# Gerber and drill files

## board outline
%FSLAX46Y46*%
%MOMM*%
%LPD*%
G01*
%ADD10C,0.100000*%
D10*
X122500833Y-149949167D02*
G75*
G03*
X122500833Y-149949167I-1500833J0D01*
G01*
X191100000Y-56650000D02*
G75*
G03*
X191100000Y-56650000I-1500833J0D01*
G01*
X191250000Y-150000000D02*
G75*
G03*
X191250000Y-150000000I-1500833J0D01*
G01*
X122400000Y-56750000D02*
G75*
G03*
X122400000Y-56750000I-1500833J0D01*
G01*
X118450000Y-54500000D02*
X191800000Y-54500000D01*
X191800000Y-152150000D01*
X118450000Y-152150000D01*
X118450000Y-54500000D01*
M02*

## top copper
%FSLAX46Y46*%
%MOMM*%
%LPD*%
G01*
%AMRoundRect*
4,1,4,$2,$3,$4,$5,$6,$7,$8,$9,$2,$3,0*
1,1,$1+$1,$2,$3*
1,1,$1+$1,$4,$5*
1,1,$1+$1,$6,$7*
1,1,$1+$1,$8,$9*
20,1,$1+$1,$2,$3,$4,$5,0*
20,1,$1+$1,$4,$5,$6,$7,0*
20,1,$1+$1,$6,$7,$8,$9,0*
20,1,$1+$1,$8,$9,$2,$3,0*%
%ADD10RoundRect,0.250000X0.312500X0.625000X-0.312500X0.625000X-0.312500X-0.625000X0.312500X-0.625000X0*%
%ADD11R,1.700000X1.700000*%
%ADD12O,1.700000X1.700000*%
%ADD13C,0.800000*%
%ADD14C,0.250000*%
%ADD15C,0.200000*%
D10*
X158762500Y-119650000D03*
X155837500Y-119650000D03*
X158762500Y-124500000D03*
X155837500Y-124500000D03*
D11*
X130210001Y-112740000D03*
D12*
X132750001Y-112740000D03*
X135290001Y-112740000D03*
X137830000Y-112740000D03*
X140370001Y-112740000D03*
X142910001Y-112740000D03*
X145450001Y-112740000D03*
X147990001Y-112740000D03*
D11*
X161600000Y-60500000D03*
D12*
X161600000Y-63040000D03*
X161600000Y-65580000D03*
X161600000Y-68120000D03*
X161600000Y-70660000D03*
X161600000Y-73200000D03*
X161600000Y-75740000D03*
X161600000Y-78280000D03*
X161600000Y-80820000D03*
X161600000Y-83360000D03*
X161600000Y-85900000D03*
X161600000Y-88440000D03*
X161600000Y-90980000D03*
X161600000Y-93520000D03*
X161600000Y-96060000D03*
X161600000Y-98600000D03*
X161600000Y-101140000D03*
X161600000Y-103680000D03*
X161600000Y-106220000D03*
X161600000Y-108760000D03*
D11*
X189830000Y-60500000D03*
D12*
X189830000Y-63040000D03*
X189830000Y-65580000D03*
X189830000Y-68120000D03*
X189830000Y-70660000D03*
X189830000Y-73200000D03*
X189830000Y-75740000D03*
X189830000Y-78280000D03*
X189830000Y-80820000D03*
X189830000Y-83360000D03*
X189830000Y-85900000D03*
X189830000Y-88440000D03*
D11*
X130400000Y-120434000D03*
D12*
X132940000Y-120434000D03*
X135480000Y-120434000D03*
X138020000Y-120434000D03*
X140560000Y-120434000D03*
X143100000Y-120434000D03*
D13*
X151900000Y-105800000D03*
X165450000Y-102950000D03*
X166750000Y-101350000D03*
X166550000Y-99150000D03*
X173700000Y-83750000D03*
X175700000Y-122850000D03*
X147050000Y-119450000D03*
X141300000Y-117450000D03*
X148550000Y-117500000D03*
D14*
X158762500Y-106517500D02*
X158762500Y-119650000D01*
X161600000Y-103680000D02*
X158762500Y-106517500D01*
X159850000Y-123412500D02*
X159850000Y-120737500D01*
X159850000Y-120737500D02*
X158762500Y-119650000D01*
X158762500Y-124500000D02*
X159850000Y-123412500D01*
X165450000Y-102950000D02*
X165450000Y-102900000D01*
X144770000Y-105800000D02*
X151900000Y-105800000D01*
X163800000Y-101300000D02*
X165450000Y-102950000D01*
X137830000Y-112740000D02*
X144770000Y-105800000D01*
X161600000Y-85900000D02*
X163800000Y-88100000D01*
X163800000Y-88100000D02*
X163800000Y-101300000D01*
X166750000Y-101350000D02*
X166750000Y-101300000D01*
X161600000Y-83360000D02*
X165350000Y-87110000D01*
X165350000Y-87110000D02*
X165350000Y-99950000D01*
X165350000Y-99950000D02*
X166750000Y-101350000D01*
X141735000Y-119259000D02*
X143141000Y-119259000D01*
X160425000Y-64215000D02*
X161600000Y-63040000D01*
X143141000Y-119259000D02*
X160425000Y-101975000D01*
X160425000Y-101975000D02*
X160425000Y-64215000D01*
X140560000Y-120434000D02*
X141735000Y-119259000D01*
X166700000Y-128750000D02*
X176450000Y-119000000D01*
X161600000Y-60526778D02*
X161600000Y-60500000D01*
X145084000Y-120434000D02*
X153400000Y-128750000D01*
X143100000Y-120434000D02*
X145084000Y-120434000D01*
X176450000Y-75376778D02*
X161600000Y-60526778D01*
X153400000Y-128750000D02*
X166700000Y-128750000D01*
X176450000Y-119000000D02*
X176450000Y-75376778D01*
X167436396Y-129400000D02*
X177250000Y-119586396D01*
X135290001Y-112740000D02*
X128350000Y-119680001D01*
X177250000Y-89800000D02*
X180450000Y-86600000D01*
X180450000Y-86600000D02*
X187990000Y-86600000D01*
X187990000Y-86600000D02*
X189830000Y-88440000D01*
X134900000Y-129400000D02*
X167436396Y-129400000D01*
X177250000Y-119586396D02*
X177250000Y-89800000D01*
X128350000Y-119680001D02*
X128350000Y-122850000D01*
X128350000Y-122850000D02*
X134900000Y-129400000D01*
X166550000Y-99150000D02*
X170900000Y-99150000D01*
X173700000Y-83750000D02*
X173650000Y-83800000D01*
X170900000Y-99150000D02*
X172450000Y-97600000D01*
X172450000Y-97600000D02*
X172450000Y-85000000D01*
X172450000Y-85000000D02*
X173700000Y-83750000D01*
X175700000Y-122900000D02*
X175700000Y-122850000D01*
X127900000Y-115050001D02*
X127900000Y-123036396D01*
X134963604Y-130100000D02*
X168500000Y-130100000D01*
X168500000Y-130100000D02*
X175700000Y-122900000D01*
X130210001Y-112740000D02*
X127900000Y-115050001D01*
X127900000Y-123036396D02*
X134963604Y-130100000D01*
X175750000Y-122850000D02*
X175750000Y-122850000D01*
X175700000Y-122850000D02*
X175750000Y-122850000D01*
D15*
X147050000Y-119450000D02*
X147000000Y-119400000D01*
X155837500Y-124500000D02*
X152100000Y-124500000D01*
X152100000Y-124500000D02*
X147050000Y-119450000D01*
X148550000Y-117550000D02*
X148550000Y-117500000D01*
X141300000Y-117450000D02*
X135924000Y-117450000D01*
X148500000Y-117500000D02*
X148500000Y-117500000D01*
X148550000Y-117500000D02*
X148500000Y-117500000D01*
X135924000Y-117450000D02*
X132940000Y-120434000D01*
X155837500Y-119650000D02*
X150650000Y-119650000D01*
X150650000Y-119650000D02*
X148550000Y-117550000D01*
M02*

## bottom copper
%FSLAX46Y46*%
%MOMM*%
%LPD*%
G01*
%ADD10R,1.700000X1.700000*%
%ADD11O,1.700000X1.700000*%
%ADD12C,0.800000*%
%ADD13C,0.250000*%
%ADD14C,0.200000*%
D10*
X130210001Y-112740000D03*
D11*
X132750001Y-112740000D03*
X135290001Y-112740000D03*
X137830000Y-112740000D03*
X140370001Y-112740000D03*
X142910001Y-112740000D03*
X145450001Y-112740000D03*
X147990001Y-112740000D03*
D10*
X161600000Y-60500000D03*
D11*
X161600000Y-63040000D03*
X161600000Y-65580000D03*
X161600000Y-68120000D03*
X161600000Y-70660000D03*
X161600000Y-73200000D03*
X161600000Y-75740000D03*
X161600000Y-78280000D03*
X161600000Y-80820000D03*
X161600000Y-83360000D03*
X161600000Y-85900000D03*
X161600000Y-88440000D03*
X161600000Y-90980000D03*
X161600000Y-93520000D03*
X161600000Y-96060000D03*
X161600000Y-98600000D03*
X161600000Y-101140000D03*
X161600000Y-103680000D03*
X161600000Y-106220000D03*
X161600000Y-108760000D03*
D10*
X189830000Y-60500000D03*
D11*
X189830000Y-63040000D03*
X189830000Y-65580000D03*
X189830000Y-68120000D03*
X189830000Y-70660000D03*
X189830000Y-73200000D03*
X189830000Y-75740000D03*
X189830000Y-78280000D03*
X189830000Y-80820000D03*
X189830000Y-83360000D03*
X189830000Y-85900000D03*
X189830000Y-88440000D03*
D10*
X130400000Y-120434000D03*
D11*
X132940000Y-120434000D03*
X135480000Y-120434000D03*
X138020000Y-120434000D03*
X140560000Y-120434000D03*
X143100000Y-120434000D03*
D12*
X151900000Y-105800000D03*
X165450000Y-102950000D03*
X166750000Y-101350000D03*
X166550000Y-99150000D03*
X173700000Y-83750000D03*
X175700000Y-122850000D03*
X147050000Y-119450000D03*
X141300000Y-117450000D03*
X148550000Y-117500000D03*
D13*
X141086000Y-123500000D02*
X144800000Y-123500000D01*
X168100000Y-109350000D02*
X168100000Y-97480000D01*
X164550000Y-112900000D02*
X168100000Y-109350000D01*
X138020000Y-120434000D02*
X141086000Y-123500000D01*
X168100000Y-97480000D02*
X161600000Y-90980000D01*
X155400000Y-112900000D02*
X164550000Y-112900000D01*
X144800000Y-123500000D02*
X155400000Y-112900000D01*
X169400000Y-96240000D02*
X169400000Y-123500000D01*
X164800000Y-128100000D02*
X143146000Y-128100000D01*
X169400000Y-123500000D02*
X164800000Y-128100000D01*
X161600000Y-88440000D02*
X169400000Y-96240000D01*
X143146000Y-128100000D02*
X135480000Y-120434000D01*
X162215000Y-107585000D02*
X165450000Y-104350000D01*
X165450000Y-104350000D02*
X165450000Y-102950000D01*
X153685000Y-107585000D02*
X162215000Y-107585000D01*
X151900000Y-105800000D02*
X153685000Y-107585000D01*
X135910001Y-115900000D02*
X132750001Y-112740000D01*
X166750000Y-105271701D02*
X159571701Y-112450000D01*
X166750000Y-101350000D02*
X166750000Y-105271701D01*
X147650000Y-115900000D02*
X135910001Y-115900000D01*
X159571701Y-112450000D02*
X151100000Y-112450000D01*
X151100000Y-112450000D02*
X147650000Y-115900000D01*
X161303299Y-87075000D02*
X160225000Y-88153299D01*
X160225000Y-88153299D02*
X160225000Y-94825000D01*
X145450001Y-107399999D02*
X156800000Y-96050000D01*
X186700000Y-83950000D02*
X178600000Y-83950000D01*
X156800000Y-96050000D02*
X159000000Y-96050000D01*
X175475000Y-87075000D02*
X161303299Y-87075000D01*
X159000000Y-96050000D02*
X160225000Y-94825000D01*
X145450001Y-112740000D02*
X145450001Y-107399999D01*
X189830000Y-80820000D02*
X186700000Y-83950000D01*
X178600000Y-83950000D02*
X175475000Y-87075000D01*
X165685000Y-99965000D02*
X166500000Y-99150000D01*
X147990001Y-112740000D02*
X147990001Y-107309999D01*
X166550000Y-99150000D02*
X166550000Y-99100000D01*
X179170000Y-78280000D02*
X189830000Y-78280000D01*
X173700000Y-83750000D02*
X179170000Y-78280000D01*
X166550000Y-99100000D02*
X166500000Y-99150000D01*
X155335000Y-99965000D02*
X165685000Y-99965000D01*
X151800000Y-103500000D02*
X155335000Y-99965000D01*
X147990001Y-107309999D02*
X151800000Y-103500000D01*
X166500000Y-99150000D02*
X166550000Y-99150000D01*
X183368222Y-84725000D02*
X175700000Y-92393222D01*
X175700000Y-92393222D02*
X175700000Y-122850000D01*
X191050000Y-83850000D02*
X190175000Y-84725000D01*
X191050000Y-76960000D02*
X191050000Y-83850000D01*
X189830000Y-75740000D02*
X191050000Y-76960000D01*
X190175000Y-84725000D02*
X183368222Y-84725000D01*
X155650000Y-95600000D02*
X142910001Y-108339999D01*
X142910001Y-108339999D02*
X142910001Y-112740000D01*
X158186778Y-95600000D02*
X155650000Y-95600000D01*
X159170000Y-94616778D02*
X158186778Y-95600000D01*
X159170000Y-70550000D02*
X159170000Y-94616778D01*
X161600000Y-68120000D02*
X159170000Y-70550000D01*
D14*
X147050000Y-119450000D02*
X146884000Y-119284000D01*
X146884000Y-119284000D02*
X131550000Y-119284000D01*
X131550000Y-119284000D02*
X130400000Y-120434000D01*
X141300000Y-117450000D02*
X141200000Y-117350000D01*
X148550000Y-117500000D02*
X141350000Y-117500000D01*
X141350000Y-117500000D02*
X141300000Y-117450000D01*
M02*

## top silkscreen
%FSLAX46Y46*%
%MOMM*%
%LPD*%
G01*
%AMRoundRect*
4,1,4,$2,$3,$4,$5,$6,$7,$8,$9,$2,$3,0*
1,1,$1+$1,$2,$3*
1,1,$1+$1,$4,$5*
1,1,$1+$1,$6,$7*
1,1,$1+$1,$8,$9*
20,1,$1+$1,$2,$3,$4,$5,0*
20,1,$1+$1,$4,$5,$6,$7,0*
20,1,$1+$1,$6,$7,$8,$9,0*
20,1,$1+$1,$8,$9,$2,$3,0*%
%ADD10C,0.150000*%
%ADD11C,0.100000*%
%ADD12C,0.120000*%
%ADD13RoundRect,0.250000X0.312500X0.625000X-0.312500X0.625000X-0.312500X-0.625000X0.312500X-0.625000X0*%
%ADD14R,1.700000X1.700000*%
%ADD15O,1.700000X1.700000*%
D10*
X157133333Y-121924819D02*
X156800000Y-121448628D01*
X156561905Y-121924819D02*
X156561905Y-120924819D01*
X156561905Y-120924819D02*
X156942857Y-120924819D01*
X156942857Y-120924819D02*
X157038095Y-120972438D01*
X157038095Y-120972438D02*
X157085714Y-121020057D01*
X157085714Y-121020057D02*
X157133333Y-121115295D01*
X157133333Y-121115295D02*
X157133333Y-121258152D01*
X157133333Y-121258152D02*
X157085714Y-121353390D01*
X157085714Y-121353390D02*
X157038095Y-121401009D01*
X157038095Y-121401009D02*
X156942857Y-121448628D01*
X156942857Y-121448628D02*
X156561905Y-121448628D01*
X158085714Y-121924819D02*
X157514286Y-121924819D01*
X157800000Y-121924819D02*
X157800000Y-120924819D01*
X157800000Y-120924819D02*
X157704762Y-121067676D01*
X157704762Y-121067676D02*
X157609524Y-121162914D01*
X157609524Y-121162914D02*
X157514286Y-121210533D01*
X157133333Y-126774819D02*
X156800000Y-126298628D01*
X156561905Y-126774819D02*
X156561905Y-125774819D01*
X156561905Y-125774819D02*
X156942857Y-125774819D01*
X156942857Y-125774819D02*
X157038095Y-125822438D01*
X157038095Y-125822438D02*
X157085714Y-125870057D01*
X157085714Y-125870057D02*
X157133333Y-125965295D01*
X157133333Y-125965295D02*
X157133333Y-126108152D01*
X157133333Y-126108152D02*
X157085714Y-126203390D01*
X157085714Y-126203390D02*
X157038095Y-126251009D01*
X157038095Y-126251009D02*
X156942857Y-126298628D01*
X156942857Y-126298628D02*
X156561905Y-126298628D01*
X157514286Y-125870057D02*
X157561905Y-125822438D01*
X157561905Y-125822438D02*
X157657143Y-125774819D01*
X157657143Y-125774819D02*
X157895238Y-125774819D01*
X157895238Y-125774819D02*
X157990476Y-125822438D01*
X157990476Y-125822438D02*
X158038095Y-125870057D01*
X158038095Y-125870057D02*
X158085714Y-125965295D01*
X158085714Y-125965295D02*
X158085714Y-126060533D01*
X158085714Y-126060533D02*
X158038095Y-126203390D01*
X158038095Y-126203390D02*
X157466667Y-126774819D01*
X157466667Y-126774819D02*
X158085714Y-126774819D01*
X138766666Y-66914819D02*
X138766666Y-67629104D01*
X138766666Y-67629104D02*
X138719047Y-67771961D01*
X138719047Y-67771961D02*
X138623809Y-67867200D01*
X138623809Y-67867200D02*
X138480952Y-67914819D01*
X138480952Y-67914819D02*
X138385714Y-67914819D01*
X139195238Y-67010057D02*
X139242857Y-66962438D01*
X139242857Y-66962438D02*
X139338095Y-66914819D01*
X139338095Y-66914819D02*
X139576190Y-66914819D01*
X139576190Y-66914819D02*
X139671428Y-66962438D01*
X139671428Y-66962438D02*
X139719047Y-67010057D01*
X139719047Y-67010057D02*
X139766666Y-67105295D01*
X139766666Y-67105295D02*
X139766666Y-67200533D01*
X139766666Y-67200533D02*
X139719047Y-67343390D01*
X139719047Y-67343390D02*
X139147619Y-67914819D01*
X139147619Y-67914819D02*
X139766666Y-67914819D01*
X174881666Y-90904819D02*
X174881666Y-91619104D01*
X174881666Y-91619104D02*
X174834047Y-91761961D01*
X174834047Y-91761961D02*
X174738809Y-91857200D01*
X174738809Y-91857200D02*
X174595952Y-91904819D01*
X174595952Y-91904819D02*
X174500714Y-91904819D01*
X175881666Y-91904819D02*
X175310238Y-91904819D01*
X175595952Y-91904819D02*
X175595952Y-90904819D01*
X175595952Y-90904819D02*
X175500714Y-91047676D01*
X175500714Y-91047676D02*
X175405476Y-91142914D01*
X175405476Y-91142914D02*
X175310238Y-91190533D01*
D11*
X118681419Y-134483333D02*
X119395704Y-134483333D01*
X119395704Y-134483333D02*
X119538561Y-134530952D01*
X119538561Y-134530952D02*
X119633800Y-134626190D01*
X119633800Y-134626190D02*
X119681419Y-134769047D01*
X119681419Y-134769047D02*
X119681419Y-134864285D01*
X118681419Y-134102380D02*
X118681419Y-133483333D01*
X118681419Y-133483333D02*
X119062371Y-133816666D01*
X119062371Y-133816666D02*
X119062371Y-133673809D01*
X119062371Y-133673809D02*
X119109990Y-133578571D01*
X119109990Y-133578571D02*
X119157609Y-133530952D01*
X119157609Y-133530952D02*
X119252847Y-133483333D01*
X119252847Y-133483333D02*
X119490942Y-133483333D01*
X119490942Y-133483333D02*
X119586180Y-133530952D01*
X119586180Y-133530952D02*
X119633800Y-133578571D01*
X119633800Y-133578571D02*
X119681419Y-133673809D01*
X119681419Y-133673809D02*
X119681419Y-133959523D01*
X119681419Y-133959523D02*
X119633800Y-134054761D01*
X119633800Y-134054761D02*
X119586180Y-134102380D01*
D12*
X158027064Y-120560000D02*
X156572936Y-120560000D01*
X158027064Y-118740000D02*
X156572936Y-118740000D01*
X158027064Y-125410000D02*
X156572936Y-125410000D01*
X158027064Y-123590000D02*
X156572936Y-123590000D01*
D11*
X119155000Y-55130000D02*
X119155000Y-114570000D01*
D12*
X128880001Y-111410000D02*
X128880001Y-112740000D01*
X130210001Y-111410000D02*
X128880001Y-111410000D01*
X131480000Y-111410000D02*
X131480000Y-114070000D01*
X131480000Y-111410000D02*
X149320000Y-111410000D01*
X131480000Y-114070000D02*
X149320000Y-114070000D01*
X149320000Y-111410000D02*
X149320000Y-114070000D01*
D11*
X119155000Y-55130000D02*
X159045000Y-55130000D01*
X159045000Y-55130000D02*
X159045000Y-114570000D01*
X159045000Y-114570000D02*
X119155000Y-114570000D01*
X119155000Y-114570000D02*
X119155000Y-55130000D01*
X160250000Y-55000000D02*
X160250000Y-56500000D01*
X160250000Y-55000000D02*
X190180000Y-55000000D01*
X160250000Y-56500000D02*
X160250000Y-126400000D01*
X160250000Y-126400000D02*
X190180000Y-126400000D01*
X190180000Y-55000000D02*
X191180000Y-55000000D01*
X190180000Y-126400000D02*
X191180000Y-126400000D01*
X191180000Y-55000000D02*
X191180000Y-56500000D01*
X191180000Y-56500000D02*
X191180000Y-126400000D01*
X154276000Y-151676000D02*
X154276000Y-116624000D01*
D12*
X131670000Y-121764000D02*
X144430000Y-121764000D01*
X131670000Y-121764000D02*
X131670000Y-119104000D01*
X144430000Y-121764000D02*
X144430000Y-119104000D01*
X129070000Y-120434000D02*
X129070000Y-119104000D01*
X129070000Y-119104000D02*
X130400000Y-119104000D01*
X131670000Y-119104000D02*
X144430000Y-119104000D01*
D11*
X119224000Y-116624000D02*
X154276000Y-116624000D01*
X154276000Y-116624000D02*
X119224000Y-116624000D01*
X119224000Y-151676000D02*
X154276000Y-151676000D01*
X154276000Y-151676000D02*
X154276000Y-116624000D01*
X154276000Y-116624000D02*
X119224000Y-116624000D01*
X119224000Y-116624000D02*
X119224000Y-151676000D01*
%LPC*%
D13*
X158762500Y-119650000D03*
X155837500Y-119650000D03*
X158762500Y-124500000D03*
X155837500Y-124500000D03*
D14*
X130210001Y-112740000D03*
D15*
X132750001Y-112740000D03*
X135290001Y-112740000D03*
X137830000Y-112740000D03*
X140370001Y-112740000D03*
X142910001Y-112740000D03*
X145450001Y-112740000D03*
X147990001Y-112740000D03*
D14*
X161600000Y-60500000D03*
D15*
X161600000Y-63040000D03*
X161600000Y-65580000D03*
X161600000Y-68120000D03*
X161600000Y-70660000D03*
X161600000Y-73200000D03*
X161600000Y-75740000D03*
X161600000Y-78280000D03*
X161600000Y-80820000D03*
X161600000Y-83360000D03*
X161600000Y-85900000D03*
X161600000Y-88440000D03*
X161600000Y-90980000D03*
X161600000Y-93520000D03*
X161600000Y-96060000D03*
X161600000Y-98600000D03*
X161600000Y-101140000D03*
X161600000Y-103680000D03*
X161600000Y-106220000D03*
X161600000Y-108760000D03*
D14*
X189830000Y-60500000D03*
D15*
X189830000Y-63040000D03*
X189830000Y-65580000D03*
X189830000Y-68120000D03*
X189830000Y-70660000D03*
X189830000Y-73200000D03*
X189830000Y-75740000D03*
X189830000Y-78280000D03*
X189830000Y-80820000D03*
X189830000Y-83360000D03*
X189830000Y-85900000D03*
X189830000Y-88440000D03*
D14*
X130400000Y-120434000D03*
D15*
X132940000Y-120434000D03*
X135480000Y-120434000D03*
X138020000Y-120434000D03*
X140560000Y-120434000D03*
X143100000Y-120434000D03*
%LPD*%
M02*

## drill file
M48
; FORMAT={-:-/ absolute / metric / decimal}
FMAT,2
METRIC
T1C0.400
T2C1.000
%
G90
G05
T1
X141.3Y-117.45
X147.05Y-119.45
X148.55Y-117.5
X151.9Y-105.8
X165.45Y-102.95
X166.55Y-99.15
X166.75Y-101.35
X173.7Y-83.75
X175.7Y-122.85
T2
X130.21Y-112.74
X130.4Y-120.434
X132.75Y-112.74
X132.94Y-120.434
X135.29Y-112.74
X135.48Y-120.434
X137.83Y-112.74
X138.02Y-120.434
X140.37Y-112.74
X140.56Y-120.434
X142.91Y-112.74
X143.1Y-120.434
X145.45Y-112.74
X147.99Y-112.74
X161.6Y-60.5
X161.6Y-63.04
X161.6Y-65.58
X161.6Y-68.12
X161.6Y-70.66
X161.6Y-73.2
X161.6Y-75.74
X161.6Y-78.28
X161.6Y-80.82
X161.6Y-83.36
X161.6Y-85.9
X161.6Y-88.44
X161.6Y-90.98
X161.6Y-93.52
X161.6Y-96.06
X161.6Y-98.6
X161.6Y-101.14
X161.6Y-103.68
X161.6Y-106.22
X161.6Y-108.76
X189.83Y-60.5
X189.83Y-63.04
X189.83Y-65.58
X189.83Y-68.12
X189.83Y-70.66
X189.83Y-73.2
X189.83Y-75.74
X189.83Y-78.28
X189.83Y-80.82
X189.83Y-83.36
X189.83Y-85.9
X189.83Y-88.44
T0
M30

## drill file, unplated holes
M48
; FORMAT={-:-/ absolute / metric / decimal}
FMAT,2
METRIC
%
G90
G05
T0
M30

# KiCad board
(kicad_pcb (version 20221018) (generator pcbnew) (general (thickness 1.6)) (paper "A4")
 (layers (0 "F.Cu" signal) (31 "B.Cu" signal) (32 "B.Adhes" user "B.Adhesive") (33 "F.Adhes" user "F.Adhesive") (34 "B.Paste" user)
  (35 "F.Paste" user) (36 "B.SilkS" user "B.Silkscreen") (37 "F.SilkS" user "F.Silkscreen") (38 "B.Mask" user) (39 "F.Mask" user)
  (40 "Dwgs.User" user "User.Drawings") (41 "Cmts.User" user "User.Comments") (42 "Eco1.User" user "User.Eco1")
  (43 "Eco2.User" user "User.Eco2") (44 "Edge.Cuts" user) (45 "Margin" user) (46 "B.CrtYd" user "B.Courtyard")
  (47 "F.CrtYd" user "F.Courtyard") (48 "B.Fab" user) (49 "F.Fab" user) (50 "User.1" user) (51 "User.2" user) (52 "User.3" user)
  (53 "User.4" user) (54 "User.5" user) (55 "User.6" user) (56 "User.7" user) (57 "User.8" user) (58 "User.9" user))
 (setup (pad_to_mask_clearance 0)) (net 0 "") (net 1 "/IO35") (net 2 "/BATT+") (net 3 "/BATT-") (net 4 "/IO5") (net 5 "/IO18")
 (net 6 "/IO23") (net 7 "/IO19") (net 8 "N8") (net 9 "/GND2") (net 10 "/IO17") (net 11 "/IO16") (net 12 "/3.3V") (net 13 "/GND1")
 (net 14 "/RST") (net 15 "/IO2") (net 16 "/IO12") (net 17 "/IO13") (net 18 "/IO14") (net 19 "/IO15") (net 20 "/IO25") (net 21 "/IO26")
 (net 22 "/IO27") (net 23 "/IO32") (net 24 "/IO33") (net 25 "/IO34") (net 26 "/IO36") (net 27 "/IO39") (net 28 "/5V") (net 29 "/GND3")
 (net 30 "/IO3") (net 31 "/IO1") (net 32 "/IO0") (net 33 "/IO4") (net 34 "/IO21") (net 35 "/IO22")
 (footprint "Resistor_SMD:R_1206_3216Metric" (layer "F.Cu") (at 157.3 119.65 180)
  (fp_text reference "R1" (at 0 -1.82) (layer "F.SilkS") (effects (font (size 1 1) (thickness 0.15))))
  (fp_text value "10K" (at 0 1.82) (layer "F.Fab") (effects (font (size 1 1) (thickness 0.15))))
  (fp_line (start -0.727064 -0.91) (end 0.727064 -0.91) (stroke (width 0.12) (type solid)) (layer "F.SilkS"))
  (fp_line (start -0.727064 0.91) (end 0.727064 0.91) (stroke (width 0.12) (type solid)) (layer "F.SilkS"))
  (pad "1" smd roundrect (at -1.4625 0 180) (size 1.125 1.75) (layers "F.Cu" "F.Paste" "F.Mask") (roundrect_rratio 0.2222222222)
   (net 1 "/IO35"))
  (pad "2" smd roundrect (at 1.4625 0 180) (size 1.125 1.75) (layers "F.Cu" "F.Paste" "F.Mask") (roundrect_rratio 0.2222222222)
   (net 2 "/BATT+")))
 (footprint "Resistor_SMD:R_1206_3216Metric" (layer "F.Cu") (at 157.3 124.5 180)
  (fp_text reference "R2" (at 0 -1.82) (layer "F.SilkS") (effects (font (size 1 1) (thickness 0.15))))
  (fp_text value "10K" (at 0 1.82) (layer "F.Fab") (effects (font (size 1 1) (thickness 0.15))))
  (fp_line (start -0.727064 -0.91) (end 0.727064 -0.91) (stroke (width 0.12) (type solid)) (layer "F.SilkS"))
  (fp_line (start -0.727064 0.91) (end 0.727064 0.91) (stroke (width 0.12) (type solid)) (layer "F.SilkS"))
  (pad "1" smd roundrect (at -1.4625 0 180) (size 1.125 1.75) (layers "F.Cu" "F.Paste" "F.Mask") (roundrect_rratio 0.2222222222)
   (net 1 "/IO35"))
  (pad "2" smd roundrect (at 1.4625 0 180) (size 1.125 1.75) (layers "F.Cu" "F.Paste" "F.Mask") (roundrect_rratio 0.2222222222)
   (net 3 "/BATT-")))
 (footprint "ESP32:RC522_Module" (layer "F.Cu") (at 139.1 84.85)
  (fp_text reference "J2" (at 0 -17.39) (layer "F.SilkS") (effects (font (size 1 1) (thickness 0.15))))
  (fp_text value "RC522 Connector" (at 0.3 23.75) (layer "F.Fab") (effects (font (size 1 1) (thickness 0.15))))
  (fp_line (start -19.945 -29.72) (end -19.945 29.72) (stroke (width 0.1) (type default)) (layer "F.SilkS"))
  (fp_line (start -10.219999 26.56) (end -10.219999 27.89) (stroke (width 0.12) (type solid)) (layer "F.SilkS"))
  (fp_line (start -8.889999 26.56) (end -10.219999 26.56) (stroke (width 0.12) (type solid)) (layer "F.SilkS"))
  (fp_line (start -7.62 26.56) (end -7.62 29.22) (stroke (width 0.12) (type solid)) (layer "F.SilkS"))
  (fp_line (start -7.62 26.56) (end 10.22 26.56) (stroke (width 0.12) (type solid)) (layer "F.SilkS"))
  (fp_line (start -7.62 29.22) (end 10.22 29.22) (stroke (width 0.12) (type solid)) (layer "F.SilkS"))
  (fp_line (start 10.22 26.56) (end 10.22 29.22) (stroke (width 0.12) (type solid)) (layer "F.SilkS"))
  (fp_rect (start -19.945 -29.72) (end 19.945 29.72) (stroke (width 0.1) (type default)) (fill none) (layer "F.SilkS"))
  (pad "1" thru_hole rect (at -8.889999 27.89 90) (size 1.7 1.7) (drill 1) (layers "*.Cu" "*.Mask") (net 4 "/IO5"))
  (pad "2" thru_hole oval (at -6.349999 27.89 90) (size 1.7 1.7) (drill 1) (layers "*.Cu" "*.Mask") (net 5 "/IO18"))
  (pad "3" thru_hole oval (at -3.809999 27.89 90) (size 1.7 1.7) (drill 1) (layers "*.Cu" "*.Mask") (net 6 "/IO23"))
  (pad "4" thru_hole oval (at -1.27 27.89 90) (size 1.7 1.7) (drill 1) (layers "*.Cu" "*.Mask") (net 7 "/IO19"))
  (pad "5" thru_hole oval (at 1.270001 27.89 90) (size 1.7 1.7) (drill 1) (layers "*.Cu" "*.Mask") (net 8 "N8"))
  (pad "6" thru_hole oval (at 3.810001 27.89 90) (size 1.7 1.7) (drill 1) (layers "*.Cu" "*.Mask") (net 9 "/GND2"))
  (pad "7" thru_hole oval (at 6.350001 27.89 90) (size 1.7 1.7) (drill 1) (layers "*.Cu" "*.Mask") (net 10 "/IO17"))
  (pad "8" thru_hole oval (at 8.890001 27.89 90) (size 1.7 1.7) (drill 1) (layers "*.Cu" "*.Mask") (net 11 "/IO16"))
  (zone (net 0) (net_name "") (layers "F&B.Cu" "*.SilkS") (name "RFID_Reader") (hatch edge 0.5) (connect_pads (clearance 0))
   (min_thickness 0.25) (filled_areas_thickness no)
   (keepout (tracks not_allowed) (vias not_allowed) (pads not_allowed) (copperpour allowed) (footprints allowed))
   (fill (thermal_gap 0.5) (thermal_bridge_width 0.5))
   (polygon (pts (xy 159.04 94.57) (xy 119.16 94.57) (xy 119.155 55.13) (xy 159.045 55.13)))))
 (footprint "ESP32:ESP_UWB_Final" (layer "F.Cu") (at 177.85 84.6)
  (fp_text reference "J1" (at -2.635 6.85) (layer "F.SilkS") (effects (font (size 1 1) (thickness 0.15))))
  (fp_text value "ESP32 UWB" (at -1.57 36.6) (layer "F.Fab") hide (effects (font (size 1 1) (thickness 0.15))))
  (fp_line (start -17.6 -29.6) (end -17.6 -28.1) (stroke (width 0.1) (type default)) (layer "F.SilkS"))
  (fp_line (start -17.6 -29.6) (end 12.33 -29.6) (stroke (width 0.1) (type default)) (layer "F.SilkS"))
  (fp_line (start -17.6 -28.1) (end -17.6 41.8) (stroke (width 0.1) (type default)) (layer "F.SilkS"))
  (fp_line (start -17.6 41.8) (end 12.33 41.8) (stroke (width 0.1) (type default)) (layer "F.SilkS"))
  (fp_line (start 12.33 -29.6) (end 13.33 -29.6) (stroke (width 0.1) (type default)) (layer "F.SilkS"))
  (fp_line (start 12.33 41.8) (end 13.33 41.8) (stroke (width 0.1) (type default)) (layer "F.SilkS"))
  (fp_line (start 13.33 -29.6) (end 13.33 -28.1) (stroke (width 0.1) (type default)) (layer "F.SilkS"))
  (fp_line (start 13.33 -28.1) (end 13.33 41.8) (stroke (width 0.1) (type default)) (layer "F.SilkS"))
  (pad "1" thru_hole rect (at -16.25 -24.1) (size 1.7 1.7) (drill 1) (layers "*.Cu" "*.Mask") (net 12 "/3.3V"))
  (pad "2" thru_hole oval (at -16.25 -21.56) (size 1.7 1.7) (drill 1) (layers "*.Cu" "*.Mask") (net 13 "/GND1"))
  (pad "3" thru_hole oval (at -16.25 -19.02) (size 1.7 1.7) (drill 1) (layers "*.Cu" "*.Mask") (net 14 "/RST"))
  (pad "4" thru_hole oval (at -16.25 -16.48) (size 1.7 1.7) (drill 1) (layers "*.Cu" "*.Mask") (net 9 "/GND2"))
  (pad "5" thru_hole oval (at -16.25 -13.94) (size 1.7 1.7) (drill 1) (layers "*.Cu" "*.Mask") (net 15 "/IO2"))
  (pad "6" thru_hole oval (at -16.25 -11.4) (size 1.7 1.7) (drill 1) (layers "*.Cu" "*.Mask") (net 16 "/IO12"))
  (pad "7" thru_hole oval (at -16.25 -8.86) (size 1.7 1.7) (drill 1) (layers "*.Cu" "*.Mask") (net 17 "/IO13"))
  (pad "8" thru_hole oval (at -16.25 -6.32) (size 1.7 1.7) (drill 1) (layers "*.Cu" "*.Mask") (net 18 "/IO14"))
  (pad "9" thru_hole oval (at -16.25 -3.78) (size 1.7 1.7) (drill 1) (layers "*.Cu" "*.Mask") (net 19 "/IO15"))
  (pad "10" thru_hole oval (at -16.25 -1.24) (size 1.7 1.7) (drill 1) (layers "*.Cu" "*.Mask") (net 5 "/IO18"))
  (pad "11" thru_hole oval (at -16.25 1.3) (size 1.7 1.7) (drill 1) (layers "*.Cu" "*.Mask") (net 7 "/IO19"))
  (pad "12" thru_hole oval (at -16.25 3.84) (size 1.7 1.7) (drill 1) (layers "*.Cu" "*.Mask") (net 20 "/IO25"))
  (pad "13" thru_hole oval (at -16.25 6.38) (size 1.7 1.7) (drill 1) (layers "*.Cu" "*.Mask") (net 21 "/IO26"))
  (pad "14" thru_hole oval (at -16.25 8.92) (size 1.7 1.7) (drill 1) (layers "*.Cu" "*.Mask") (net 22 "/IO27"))
  (pad "15" thru_hole oval (at -16.25 11.46) (size 1.7 1.7) (drill 1) (layers "*.Cu" "*.Mask") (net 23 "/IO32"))
  (pad "16" thru_hole oval (at -16.25 14) (size 1.7 1.7) (drill 1) (layers "*.Cu" "*.Mask") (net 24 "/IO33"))
  (pad "17" thru_hole oval (at -16.25 16.54) (size 1.7 1.7) (drill 1) (layers "*.Cu" "*.Mask") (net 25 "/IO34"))
  (pad "18" thru_hole oval (at -16.25 19.08) (size 1.7 1.7) (drill 1) (layers "*.Cu" "*.Mask") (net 1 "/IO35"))
  (pad "19" thru_hole oval (at -16.25 21.62) (size 1.7 1.7) (drill 1) (layers "*.Cu" "*.Mask") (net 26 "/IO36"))
  (pad "20" thru_hole oval (at -16.25 24.16) (size 1.7 1.7) (drill 1) (layers "*.Cu" "*.Mask") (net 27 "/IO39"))
  (pad "21" thru_hole rect (at 11.98 -24.1) (size 1.7 1.7) (drill 1) (layers "*.Cu" "*.Mask") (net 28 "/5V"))
  (pad "22" thru_hole oval (at 11.98 -21.56) (size 1.7 1.7) (drill 1) (layers "*.Cu" "*.Mask") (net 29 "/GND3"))
  (pad "23" thru_hole oval (at 11.98 -19.02) (size 1.7 1.7) (drill 1) (layers "*.Cu" "*.Mask") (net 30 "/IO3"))
  (pad "24" thru_hole oval (at 11.98 -16.48) (size 1.7 1.7) (drill 1) (layers "*.Cu" "*.Mask") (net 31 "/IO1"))
  (pad "25" thru_hole oval (at 11.98 -13.94) (size 1.7 1.7) (drill 1) (layers "*.Cu" "*.Mask") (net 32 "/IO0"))
  (pad "26" thru_hole oval (at 11.98 -11.4) (size 1.7 1.7) (drill 1) (layers "*.Cu" "*.Mask") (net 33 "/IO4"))
  (pad "27" thru_hole oval (at 11.98 -8.86) (size 1.7 1.7) (drill 1) (layers "*.Cu" "*.Mask") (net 4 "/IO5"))
  (pad "28" thru_hole oval (at 11.98 -6.32) (size 1.7 1.7) (drill 1) (layers "*.Cu" "*.Mask") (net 11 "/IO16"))
  (pad "29" thru_hole oval (at 11.98 -3.78) (size 1.7 1.7) (drill 1) (layers "*.Cu" "*.Mask") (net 10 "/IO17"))
  (pad "30" thru_hole oval (at 11.98 -1.24) (size 1.7 1.7) (drill 1) (layers "*.Cu" "*.Mask") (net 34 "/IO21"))
  (pad "31" thru_hole oval (at 11.98 1.3) (size 1.7 1.7) (drill 1) (layers "*.Cu" "*.Mask") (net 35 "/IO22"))
  (pad "32" thru_hole oval (at 11.98 3.84) (size 1.7 1.7) (drill 1) (layers "*.Cu" "*.Mask") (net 6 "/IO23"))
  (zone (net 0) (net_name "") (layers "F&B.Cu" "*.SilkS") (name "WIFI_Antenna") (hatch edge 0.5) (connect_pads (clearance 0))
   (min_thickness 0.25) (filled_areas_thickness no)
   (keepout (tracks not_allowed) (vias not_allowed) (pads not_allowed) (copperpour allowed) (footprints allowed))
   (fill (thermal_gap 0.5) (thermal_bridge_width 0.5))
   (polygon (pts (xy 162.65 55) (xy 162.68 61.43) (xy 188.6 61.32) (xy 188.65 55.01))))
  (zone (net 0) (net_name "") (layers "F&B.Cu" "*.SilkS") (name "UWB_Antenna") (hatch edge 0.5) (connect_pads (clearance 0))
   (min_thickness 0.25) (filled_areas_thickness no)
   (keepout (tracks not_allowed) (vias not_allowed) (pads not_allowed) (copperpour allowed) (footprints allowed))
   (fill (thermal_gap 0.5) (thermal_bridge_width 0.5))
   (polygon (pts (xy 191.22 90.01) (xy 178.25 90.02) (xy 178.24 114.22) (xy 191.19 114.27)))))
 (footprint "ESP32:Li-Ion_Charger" (layer "F.Cu") (at 136.75 134.15 90)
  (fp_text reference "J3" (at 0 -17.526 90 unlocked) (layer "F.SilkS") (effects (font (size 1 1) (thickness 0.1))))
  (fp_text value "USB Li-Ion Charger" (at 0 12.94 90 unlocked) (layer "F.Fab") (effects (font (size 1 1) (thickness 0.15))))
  (fp_line (start -17.526 17.526) (end 17.526 17.526) (stroke (width 0.1) (type default)) (layer "F.SilkS"))
  (fp_line (start 12.386 -5.08) (end 12.386 7.68) (stroke (width 0.12) (type solid)) (layer "F.SilkS"))
  (fp_line (start 12.386 -5.08) (end 15.046 -5.08) (stroke (width 0.12) (type solid)) (layer "F.SilkS"))
  (fp_line (start 12.386 7.68) (end 15.046 7.68) (stroke (width 0.12) (type solid)) (layer "F.SilkS"))
  (fp_line (start 13.716 -7.68) (end 15.046 -7.68) (stroke (width 0.12) (type solid)) (layer "F.SilkS"))
  (fp_line (start 15.046 -7.68) (end 15.046 -6.35) (stroke (width 0.12) (type solid)) (layer "F.SilkS"))
  (fp_line (start 15.046 -5.08) (end 15.046 7.68) (stroke (width 0.12) (type solid)) (layer "F.SilkS"))
  (fp_line (start 17.526 -17.526) (end 17.526 17.526) (stroke (width 0.1) (type default)) (layer "F.SilkS"))
  (fp_line (start 17.526 17.526) (end 17.526 -17.526) (stroke (width 0.1) (type default)) (layer "F.SilkS"))
  (fp_rect (start -17.526 -17.526) (end 17.526 17.526) (stroke (width 0.1) (type default)) (fill none) (layer "F.SilkS"))
  (pad "1" thru_hole rect (at 13.716 -6.35 90) (size 1.7 1.7) (drill 1) (layers "*.Cu" "*.Mask") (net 3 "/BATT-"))
  (pad "2" thru_hole oval (at 13.716 -3.81 90) (size 1.7 1.7) (drill 1) (layers "*.Cu" "*.Mask") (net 2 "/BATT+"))
  (pad "3" thru_hole oval (at 13.716 -1.27 90) (size 1.7 1.7) (drill 1) (layers "*.Cu" "*.Mask") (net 20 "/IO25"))
  (pad "4" thru_hole oval (at 13.716 1.27 90) (size 1.7 1.7) (drill 1) (layers "*.Cu" "*.Mask") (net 21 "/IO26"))
  (pad "5" thru_hole oval (at 13.716 3.81 90) (size 1.7 1.7) (drill 1) (layers "*.Cu" "*.Mask") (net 13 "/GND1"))
  (pad "6" thru_hole oval (at 13.716 6.35 90) (size 1.7 1.7) (drill 1) (layers "*.Cu" "*.Mask") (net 12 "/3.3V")))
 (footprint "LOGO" (layer "B.Cu") (at 154.55 97.1 180)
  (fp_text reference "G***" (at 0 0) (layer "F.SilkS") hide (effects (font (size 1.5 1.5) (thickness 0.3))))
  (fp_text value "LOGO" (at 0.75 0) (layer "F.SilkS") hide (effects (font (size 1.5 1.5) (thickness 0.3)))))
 (gr_circle (center 121 149.949167) (end 119.7 149.199167) (stroke (width 0.1) (type default)) (fill none) (layer "Edge.Cuts"))
 (gr_circle (center 189.599167 56.65) (end 188.299167 55.9) (stroke (width 0.1) (type default)) (fill none) (layer "Edge.Cuts"))
 (gr_circle (center 189.749167 150) (end 188.449167 149.25) (stroke (width 0.1) (type default)) (fill none) (layer "Edge.Cuts"))
 (gr_circle (center 120.899167 56.75) (end 119.599167 56) (stroke (width 0.1) (type default)) (fill none) (layer "Edge.Cuts"))
 (gr_rect (start 118.45 54.5) (end 191.8 152.15) (stroke (width 0.1) (type default)) (fill none) (layer "Edge.Cuts"))
 (segment (start 158.7625 106.5175) (end 158.7625 119.65) (width 0.25) (layer "F.Cu") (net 1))
 (segment (start 161.6 103.68) (end 158.7625 106.5175) (width 0.25) (layer "F.Cu") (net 1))
 (segment (start 159.85 123.4125) (end 159.85 120.7375) (width 0.25) (layer "F.Cu") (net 1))
 (segment (start 159.85 120.7375) (end 158.7625 119.65) (width 0.25) (layer "F.Cu") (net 1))
 (segment (start 158.7625 124.5) (end 159.85 123.4125) (width 0.25) (layer "F.Cu") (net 1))
 (segment (start 141.086 123.5) (end 144.8 123.5) (width 0.25) (layer "B.Cu") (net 21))
 (segment (start 168.1 109.35) (end 168.1 97.48) (width 0.25) (layer "B.Cu") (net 21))
 (segment (start 164.55 112.9) (end 168.1 109.35) (width 0.25) (layer "B.Cu") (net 21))
 (segment (start 138.02 120.434) (end 141.086 123.5) (width 0.25) (layer "B.Cu") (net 21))
 (segment (start 168.1 97.48) (end 161.6 90.98) (width 0.25) (layer "B.Cu") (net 21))
 (segment (start 155.4 112.9) (end 164.55 112.9) (width 0.25) (layer "B.Cu") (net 21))
 (segment (start 144.8 123.5) (end 155.4 112.9) (width 0.25) (layer "B.Cu") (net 21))
 (segment (start 169.4 96.24) (end 169.4 123.5) (width 0.25) (layer "B.Cu") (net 20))
 (segment (start 164.8 128.1) (end 143.146 128.1) (width 0.25) (layer "B.Cu") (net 20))
 (segment (start 169.4 123.5) (end 164.8 128.1) (width 0.25) (layer "B.Cu") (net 20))
 (segment (start 161.6 88.44) (end 169.4 96.24) (width 0.25) (layer "B.Cu") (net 20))
 (segment (start 143.146 128.1) (end 135.48 120.434) (width 0.25) (layer "B.Cu") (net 20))
 (segment (start 165.45 102.95) (end 165.45 102.9) (width 0.25) (layer "F.Cu") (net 7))
 (segment (start 144.77 105.8) (end 151.9 105.8) (width 0.25) (layer "F.Cu") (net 7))
 (segment (start 163.8 101.3) (end 165.45 102.95) (width 0.25) (layer "F.Cu") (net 7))
 (segment (start 137.83 112.74) (end 144.77 105.8) (width 0.25) (layer "F.Cu") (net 7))
 (segment (start 161.6 85.9) (end 163.8 88.1) (width 0.25) (layer "F.Cu") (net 7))
 (segment (start 163.8 88.1) (end 163.8 101.3) (width 0.25) (layer "F.Cu") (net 7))
 (via (at 151.9 105.8) (size 0.8) (drill 0.4) (layers "F.Cu" "B.Cu") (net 7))
 (via (at 165.45 102.95) (size 0.8) (drill 0.4) (layers "F.Cu" "B.Cu") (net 7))
 (segment (start 162.215 107.585) (end 165.45 104.35) (width 0.25) (layer "B.Cu") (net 7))
 (segment (start 165.45 104.35) (end 165.45 102.95) (width 0.25) (layer "B.Cu") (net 7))
 (segment (start 153.685 107.585) (end 162.215 107.585) (width 0.25) (layer "B.Cu") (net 7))
 (segment (start 151.9 105.8) (end 153.685 107.585) (width 0.25) (layer "B.Cu") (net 7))
 (segment (start 166.75 101.35) (end 166.75 101.3) (width 0.25) (layer "F.Cu") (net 5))
 (segment (start 161.6 83.36) (end 165.35 87.11) (width 0.25) (layer "F.Cu") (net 5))
 (segment (start 165.35 87.11) (end 165.35 99.95) (width 0.25) (layer "F.Cu") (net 5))
 (segment (start 165.35 99.95) (end 166.75 101.35) (width 0.25) (layer "F.Cu") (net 5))
 (via (at 166.75 101.35) (size 0.8) (drill 0.4) (layers "F.Cu" "B.Cu") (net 5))
 (segment (start 135.910001 115.9) (end 132.750001 112.74) (width 0.25) (layer "B.Cu") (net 5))
 (segment (start 166.75 105.271701) (end 159.571701 112.45) (width 0.25) (layer "B.Cu") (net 5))
 (segment (start 166.75 101.35) (end 166.75 105.271701) (width 0.25) (layer "B.Cu") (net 5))
 (segment (start 147.65 115.9) (end 135.910001 115.9) (width 0.25) (layer "B.Cu") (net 5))
 (segment (start 159.571701 112.45) (end 151.1 112.45) (width 0.25) (layer "B.Cu") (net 5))
 (segment (start 151.1 112.45) (end 147.65 115.9) (width 0.25) (layer "B.Cu") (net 5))
 (segment (start 141.735 119.259) (end 143.141 119.259) (width 0.25) (layer "F.Cu") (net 13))
 (segment (start 160.425 64.215) (end 161.6 63.04) (width 0.25) (layer "F.Cu") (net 13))
 (segment (start 143.141 119.259) (end 160.425 101.975) (width 0.25) (layer "F.Cu") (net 13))
 (segment (start 160.425 101.975) (end 160.425 64.215) (width 0.25) (layer "F.Cu") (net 13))
 (segment (start 140.56 120.434) (end 141.735 119.259) (width 0.25) (layer "F.Cu") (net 13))
 (segment (start 166.7 128.75) (end 176.45 119) (width 0.25) (layer "F.Cu") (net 12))
 (segment (start 161.6 60.526778) (end 161.6 60.5) (width 0.25) (layer "F.Cu") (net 12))
 (segment (start 145.084 120.434) (end 153.4 128.75) (width 0.25) (layer "F.Cu") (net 12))
 (segment (start 143.1 120.434) (end 145.084 120.434) (width 0.25) (layer "F.Cu") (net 12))
 (segment (start 176.45 75.376778) (end 161.6 60.526778) (width 0.25) (layer "F.Cu") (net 12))
 (segment (start 153.4 128.75) (end 166.7 128.75) (width 0.25) (layer "F.Cu") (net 12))
 (segment (start 176.45 119) (end 176.45 75.376778) (width 0.25) (layer "F.Cu") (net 12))
 (segment (start 167.436396 129.4) (end 177.25 119.586396) (width 0.25) (layer "F.Cu") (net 6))
 (segment (start 135.290001 112.74) (end 128.35 119.680001) (width 0.25) (layer "F.Cu") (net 6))
 (segment (start 177.25 89.8) (end 180.45 86.6) (width 0.25) (layer "F.Cu") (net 6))
 (segment (start 180.45 86.6) (end 187.99 86.6) (width 0.25) (layer "F.Cu") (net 6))
 (segment (start 187.99 86.6) (end 189.83 88.44) (width 0.25) (layer "F.Cu") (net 6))
 (segment (start 134.9 129.4) (end 167.436396 129.4) (width 0.25) (layer "F.Cu") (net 6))
 (segment (start 177.25 119.586396) (end 177.25 89.8) (width 0.25) (layer "F.Cu") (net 6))
 (segment (start 128.35 119.680001) (end 128.35 122.85) (width 0.25) (layer "F.Cu") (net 6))
 (segment (start 128.35 122.85) (end 134.9 129.4) (width 0.25) (layer "F.Cu") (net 6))
 (segment (start 161.303299 87.075) (end 160.225 88.153299) (width 0.25) (layer "B.Cu") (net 10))
 (segment (start 160.225 88.153299) (end 160.225 94.825) (width 0.25) (layer "B.Cu") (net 10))
 (segment (start 145.450001 107.399999) (end 156.8 96.05) (width 0.25) (layer "B.Cu") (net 10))
 (segment (start 186.7 83.95) (end 178.6 83.95) (width 0.25) (layer "B.Cu") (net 10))
 (segment (start 156.8 96.05) (end 159 96.05) (width 0.25) (layer "B.Cu") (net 10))
 (segment (start 175.475 87.075) (end 161.303299 87.075) (width 0.25) (layer "B.Cu") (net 10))
 (segment (start 159 96.05) (end 160.225 94.825) (width 0.25) (layer "B.Cu") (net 10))
 (segment (start 145.450001 112.74) (end 145.450001 107.399999) (width 0.25) (layer "B.Cu") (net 10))
 (segment (start 189.83 80.82) (end 186.7 83.95) (width 0.25) (layer "B.Cu") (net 10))
 (segment (start 178.6 83.95) (end 175.475 87.075) (width 0.25) (layer "B.Cu") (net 10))
 (segment (start 166.55 99.15) (end 170.9 99.15) (width 0.25) (layer "F.Cu") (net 11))
 (segment (start 173.7 83.75) (end 173.65 83.8) (width 0.25) (layer "F.Cu") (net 11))
 (segment (start 170.9 99.15) (end 172.45 97.6) (width 0.25) (layer "F.Cu") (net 11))
 (segment (start 172.45 97.6) (end 172.45 85) (width 0.25) (layer "F.Cu") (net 11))
 (segment (start 172.45 85) (end 173.7 83.75) (width 0.25) (layer "F.Cu") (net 11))
 (via (at 166.55 99.15) (size 0.8) (drill 0.4) (layers "F.Cu" "B.Cu") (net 11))
 (via (at 173.7 83.75) (size 0.8) (drill 0.4) (layers "F.Cu" "B.Cu") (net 11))
 (segment (start 165.685 99.965) (end 166.5 99.15) (width 0.25) (layer "B.Cu") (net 11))
 (segment (start 147.990001 112.74) (end 147.990001 107.309999) (width 0.25) (layer "B.Cu") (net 11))
 (segment (start 166.55 99.15) (end 166.55 99.1) (width 0.25) (layer "B.Cu") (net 11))
 (segment (start 179.17 78.28) (end 189.83 78.28) (width 0.25) (layer "B.Cu") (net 11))
 (segment (start 173.7 83.75) (end 179.17 78.28) (width 0.25) (layer "B.Cu") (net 11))
 (segment (start 166.55 99.1) (end 166.5 99.15) (width 0.25) (layer "B.Cu") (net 11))
 (segment (start 155.335 99.965) (end 165.685 99.965) (width 0.25) (layer "B.Cu") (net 11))
 (segment (start 151.8 103.5) (end 155.335 99.965) (width 0.25) (layer "B.Cu") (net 11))
 (segment (start 147.990001 107.309999) (end 151.8 103.5) (width 0.25) (layer "B.Cu") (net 11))
 (segment (start 166.5 99.15) (end 166.55 99.15) (width 0.25) (layer "B.Cu") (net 11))
 (segment (start 175.7 122.9) (end 175.7 122.85) (width 0.25) (layer "F.Cu") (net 4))
 (segment (start 127.9 115.050001) (end 127.9 123.036396) (width 0.25) (layer "F.Cu") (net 4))
 (segment (start 134.963604 130.1) (end 168.5 130.1) (width 0.25) (layer "F.Cu") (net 4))
 (segment (start 168.5 130.1) (end 175.7 122.9) (width 0.25) (layer "F.Cu") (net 4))
 (segment (start 130.210001 112.74) (end 127.9 115.050001) (width 0.25) (layer "F.Cu") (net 4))
 (segment (start 127.9 123.036396) (end 134.963604 130.1) (width 0.25) (layer "F.Cu") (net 4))
 (segment (start 175.75 122.85) (end 175.75 122.85) (width 0.25) (layer "F.Cu") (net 4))
 (segment (start 175.7 122.85) (end 175.75 122.85) (width 0.25) (layer "F.Cu") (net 4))
 (via (at 175.7 122.85) (size 0.8) (drill 0.4) (layers "F.Cu" "B.Cu") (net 4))
 (segment (start 183.368222 84.725) (end 175.7 92.393222) (width 0.25) (layer "B.Cu") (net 4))
 (segment (start 175.7 92.393222) (end 175.7 122.85) (width 0.25) (layer "B.Cu") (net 4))
 (segment (start 191.05 83.85) (end 190.175 84.725) (width 0.25) (layer "B.Cu") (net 4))
 (segment (start 191.05 76.96) (end 191.05 83.85) (width 0.25) (layer "B.Cu") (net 4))
 (segment (start 189.83 75.74) (end 191.05 76.96) (width 0.25) (layer "B.Cu") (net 4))
 (segment (start 190.175 84.725) (end 183.368222 84.725) (width 0.25) (layer "B.Cu") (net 4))
 (segment (start 155.65 95.6) (end 142.910001 108.339999) (width 0.25) (layer "B.Cu") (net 9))
 (segment (start 142.910001 108.339999) (end 142.910001 112.74) (width 0.25) (layer "B.Cu") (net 9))
 (segment (start 158.186778 95.6) (end 155.65 95.6) (width 0.25) (layer "B.Cu") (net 9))
 (segment (start 159.17 94.616778) (end 158.186778 95.6) (width 0.25) (layer "B.Cu") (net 9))
 (segment (start 159.17 70.55) (end 159.17 94.616778) (width 0.25) (layer "B.Cu") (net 9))
 (segment (start 161.6 68.12) (end 159.17 70.55) (width 0.25) (layer "B.Cu") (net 9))
 (segment (start 147.05 119.45) (end 147 119.4) (width 0.2) (layer "F.Cu") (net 3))
 (segment (start 155.8375 124.5) (end 152.1 124.5) (width 0.2) (layer "F.Cu") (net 3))
 (segment (start 152.1 124.5) (end 147.05 119.45) (width 0.2) (layer "F.Cu") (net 3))
 (via (at 147.05 119.45) (size 0.8) (drill 0.4) (layers "F.Cu" "B.Cu") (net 3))
 (segment (start 147.05 119.45) (end 146.884 119.284) (width 0.2) (layer "B.Cu") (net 3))
 (segment (start 146.884 119.284) (end 131.55 119.284) (width 0.2) (layer "B.Cu") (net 3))
 (segment (start 131.55 119.284) (end 130.4 120.434) (width 0.2) (layer "B.Cu") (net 3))
 (segment (start 148.55 117.55) (end 148.55 117.5) (width 0.2) (layer "F.Cu") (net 2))
 (segment (start 141.3 117.45) (end 135.924 117.45) (width 0.2) (layer "F.Cu") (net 2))
 (segment (start 148.5 117.5) (end 148.5 117.5) (width 0.2) (layer "F.Cu") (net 2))
 (segment (start 148.55 117.5) (end 148.5 117.5) (width 0.2) (layer "F.Cu") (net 2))
 (segment (start 135.924 117.45) (end 132.94 120.434) (width 0.2) (layer "F.Cu") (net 2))
 (segment (start 155.8375 119.65) (end 150.65 119.65) (width 0.2) (layer "F.Cu") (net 2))
 (segment (start 150.65 119.65) (end 148.55 117.55) (width 0.2) (layer "F.Cu") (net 2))
 (via (at 141.3 117.45) (size 0.8) (drill 0.4) (layers "F.Cu" "B.Cu") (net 2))
 (via (at 148.55 117.5) (size 0.8) (drill 0.4) (layers "F.Cu" "B.Cu") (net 2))
 (segment (start 141.3 117.45) (end 141.2 117.35) (width 0.2) (layer "B.Cu") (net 2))
 (segment (start 148.55 117.5) (end 141.35 117.5) (width 0.2) (layer "B.Cu") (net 2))
 (segment (start 141.35 117.5) (end 141.3 117.45) (width 0.2) (layer "B.Cu") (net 2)))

